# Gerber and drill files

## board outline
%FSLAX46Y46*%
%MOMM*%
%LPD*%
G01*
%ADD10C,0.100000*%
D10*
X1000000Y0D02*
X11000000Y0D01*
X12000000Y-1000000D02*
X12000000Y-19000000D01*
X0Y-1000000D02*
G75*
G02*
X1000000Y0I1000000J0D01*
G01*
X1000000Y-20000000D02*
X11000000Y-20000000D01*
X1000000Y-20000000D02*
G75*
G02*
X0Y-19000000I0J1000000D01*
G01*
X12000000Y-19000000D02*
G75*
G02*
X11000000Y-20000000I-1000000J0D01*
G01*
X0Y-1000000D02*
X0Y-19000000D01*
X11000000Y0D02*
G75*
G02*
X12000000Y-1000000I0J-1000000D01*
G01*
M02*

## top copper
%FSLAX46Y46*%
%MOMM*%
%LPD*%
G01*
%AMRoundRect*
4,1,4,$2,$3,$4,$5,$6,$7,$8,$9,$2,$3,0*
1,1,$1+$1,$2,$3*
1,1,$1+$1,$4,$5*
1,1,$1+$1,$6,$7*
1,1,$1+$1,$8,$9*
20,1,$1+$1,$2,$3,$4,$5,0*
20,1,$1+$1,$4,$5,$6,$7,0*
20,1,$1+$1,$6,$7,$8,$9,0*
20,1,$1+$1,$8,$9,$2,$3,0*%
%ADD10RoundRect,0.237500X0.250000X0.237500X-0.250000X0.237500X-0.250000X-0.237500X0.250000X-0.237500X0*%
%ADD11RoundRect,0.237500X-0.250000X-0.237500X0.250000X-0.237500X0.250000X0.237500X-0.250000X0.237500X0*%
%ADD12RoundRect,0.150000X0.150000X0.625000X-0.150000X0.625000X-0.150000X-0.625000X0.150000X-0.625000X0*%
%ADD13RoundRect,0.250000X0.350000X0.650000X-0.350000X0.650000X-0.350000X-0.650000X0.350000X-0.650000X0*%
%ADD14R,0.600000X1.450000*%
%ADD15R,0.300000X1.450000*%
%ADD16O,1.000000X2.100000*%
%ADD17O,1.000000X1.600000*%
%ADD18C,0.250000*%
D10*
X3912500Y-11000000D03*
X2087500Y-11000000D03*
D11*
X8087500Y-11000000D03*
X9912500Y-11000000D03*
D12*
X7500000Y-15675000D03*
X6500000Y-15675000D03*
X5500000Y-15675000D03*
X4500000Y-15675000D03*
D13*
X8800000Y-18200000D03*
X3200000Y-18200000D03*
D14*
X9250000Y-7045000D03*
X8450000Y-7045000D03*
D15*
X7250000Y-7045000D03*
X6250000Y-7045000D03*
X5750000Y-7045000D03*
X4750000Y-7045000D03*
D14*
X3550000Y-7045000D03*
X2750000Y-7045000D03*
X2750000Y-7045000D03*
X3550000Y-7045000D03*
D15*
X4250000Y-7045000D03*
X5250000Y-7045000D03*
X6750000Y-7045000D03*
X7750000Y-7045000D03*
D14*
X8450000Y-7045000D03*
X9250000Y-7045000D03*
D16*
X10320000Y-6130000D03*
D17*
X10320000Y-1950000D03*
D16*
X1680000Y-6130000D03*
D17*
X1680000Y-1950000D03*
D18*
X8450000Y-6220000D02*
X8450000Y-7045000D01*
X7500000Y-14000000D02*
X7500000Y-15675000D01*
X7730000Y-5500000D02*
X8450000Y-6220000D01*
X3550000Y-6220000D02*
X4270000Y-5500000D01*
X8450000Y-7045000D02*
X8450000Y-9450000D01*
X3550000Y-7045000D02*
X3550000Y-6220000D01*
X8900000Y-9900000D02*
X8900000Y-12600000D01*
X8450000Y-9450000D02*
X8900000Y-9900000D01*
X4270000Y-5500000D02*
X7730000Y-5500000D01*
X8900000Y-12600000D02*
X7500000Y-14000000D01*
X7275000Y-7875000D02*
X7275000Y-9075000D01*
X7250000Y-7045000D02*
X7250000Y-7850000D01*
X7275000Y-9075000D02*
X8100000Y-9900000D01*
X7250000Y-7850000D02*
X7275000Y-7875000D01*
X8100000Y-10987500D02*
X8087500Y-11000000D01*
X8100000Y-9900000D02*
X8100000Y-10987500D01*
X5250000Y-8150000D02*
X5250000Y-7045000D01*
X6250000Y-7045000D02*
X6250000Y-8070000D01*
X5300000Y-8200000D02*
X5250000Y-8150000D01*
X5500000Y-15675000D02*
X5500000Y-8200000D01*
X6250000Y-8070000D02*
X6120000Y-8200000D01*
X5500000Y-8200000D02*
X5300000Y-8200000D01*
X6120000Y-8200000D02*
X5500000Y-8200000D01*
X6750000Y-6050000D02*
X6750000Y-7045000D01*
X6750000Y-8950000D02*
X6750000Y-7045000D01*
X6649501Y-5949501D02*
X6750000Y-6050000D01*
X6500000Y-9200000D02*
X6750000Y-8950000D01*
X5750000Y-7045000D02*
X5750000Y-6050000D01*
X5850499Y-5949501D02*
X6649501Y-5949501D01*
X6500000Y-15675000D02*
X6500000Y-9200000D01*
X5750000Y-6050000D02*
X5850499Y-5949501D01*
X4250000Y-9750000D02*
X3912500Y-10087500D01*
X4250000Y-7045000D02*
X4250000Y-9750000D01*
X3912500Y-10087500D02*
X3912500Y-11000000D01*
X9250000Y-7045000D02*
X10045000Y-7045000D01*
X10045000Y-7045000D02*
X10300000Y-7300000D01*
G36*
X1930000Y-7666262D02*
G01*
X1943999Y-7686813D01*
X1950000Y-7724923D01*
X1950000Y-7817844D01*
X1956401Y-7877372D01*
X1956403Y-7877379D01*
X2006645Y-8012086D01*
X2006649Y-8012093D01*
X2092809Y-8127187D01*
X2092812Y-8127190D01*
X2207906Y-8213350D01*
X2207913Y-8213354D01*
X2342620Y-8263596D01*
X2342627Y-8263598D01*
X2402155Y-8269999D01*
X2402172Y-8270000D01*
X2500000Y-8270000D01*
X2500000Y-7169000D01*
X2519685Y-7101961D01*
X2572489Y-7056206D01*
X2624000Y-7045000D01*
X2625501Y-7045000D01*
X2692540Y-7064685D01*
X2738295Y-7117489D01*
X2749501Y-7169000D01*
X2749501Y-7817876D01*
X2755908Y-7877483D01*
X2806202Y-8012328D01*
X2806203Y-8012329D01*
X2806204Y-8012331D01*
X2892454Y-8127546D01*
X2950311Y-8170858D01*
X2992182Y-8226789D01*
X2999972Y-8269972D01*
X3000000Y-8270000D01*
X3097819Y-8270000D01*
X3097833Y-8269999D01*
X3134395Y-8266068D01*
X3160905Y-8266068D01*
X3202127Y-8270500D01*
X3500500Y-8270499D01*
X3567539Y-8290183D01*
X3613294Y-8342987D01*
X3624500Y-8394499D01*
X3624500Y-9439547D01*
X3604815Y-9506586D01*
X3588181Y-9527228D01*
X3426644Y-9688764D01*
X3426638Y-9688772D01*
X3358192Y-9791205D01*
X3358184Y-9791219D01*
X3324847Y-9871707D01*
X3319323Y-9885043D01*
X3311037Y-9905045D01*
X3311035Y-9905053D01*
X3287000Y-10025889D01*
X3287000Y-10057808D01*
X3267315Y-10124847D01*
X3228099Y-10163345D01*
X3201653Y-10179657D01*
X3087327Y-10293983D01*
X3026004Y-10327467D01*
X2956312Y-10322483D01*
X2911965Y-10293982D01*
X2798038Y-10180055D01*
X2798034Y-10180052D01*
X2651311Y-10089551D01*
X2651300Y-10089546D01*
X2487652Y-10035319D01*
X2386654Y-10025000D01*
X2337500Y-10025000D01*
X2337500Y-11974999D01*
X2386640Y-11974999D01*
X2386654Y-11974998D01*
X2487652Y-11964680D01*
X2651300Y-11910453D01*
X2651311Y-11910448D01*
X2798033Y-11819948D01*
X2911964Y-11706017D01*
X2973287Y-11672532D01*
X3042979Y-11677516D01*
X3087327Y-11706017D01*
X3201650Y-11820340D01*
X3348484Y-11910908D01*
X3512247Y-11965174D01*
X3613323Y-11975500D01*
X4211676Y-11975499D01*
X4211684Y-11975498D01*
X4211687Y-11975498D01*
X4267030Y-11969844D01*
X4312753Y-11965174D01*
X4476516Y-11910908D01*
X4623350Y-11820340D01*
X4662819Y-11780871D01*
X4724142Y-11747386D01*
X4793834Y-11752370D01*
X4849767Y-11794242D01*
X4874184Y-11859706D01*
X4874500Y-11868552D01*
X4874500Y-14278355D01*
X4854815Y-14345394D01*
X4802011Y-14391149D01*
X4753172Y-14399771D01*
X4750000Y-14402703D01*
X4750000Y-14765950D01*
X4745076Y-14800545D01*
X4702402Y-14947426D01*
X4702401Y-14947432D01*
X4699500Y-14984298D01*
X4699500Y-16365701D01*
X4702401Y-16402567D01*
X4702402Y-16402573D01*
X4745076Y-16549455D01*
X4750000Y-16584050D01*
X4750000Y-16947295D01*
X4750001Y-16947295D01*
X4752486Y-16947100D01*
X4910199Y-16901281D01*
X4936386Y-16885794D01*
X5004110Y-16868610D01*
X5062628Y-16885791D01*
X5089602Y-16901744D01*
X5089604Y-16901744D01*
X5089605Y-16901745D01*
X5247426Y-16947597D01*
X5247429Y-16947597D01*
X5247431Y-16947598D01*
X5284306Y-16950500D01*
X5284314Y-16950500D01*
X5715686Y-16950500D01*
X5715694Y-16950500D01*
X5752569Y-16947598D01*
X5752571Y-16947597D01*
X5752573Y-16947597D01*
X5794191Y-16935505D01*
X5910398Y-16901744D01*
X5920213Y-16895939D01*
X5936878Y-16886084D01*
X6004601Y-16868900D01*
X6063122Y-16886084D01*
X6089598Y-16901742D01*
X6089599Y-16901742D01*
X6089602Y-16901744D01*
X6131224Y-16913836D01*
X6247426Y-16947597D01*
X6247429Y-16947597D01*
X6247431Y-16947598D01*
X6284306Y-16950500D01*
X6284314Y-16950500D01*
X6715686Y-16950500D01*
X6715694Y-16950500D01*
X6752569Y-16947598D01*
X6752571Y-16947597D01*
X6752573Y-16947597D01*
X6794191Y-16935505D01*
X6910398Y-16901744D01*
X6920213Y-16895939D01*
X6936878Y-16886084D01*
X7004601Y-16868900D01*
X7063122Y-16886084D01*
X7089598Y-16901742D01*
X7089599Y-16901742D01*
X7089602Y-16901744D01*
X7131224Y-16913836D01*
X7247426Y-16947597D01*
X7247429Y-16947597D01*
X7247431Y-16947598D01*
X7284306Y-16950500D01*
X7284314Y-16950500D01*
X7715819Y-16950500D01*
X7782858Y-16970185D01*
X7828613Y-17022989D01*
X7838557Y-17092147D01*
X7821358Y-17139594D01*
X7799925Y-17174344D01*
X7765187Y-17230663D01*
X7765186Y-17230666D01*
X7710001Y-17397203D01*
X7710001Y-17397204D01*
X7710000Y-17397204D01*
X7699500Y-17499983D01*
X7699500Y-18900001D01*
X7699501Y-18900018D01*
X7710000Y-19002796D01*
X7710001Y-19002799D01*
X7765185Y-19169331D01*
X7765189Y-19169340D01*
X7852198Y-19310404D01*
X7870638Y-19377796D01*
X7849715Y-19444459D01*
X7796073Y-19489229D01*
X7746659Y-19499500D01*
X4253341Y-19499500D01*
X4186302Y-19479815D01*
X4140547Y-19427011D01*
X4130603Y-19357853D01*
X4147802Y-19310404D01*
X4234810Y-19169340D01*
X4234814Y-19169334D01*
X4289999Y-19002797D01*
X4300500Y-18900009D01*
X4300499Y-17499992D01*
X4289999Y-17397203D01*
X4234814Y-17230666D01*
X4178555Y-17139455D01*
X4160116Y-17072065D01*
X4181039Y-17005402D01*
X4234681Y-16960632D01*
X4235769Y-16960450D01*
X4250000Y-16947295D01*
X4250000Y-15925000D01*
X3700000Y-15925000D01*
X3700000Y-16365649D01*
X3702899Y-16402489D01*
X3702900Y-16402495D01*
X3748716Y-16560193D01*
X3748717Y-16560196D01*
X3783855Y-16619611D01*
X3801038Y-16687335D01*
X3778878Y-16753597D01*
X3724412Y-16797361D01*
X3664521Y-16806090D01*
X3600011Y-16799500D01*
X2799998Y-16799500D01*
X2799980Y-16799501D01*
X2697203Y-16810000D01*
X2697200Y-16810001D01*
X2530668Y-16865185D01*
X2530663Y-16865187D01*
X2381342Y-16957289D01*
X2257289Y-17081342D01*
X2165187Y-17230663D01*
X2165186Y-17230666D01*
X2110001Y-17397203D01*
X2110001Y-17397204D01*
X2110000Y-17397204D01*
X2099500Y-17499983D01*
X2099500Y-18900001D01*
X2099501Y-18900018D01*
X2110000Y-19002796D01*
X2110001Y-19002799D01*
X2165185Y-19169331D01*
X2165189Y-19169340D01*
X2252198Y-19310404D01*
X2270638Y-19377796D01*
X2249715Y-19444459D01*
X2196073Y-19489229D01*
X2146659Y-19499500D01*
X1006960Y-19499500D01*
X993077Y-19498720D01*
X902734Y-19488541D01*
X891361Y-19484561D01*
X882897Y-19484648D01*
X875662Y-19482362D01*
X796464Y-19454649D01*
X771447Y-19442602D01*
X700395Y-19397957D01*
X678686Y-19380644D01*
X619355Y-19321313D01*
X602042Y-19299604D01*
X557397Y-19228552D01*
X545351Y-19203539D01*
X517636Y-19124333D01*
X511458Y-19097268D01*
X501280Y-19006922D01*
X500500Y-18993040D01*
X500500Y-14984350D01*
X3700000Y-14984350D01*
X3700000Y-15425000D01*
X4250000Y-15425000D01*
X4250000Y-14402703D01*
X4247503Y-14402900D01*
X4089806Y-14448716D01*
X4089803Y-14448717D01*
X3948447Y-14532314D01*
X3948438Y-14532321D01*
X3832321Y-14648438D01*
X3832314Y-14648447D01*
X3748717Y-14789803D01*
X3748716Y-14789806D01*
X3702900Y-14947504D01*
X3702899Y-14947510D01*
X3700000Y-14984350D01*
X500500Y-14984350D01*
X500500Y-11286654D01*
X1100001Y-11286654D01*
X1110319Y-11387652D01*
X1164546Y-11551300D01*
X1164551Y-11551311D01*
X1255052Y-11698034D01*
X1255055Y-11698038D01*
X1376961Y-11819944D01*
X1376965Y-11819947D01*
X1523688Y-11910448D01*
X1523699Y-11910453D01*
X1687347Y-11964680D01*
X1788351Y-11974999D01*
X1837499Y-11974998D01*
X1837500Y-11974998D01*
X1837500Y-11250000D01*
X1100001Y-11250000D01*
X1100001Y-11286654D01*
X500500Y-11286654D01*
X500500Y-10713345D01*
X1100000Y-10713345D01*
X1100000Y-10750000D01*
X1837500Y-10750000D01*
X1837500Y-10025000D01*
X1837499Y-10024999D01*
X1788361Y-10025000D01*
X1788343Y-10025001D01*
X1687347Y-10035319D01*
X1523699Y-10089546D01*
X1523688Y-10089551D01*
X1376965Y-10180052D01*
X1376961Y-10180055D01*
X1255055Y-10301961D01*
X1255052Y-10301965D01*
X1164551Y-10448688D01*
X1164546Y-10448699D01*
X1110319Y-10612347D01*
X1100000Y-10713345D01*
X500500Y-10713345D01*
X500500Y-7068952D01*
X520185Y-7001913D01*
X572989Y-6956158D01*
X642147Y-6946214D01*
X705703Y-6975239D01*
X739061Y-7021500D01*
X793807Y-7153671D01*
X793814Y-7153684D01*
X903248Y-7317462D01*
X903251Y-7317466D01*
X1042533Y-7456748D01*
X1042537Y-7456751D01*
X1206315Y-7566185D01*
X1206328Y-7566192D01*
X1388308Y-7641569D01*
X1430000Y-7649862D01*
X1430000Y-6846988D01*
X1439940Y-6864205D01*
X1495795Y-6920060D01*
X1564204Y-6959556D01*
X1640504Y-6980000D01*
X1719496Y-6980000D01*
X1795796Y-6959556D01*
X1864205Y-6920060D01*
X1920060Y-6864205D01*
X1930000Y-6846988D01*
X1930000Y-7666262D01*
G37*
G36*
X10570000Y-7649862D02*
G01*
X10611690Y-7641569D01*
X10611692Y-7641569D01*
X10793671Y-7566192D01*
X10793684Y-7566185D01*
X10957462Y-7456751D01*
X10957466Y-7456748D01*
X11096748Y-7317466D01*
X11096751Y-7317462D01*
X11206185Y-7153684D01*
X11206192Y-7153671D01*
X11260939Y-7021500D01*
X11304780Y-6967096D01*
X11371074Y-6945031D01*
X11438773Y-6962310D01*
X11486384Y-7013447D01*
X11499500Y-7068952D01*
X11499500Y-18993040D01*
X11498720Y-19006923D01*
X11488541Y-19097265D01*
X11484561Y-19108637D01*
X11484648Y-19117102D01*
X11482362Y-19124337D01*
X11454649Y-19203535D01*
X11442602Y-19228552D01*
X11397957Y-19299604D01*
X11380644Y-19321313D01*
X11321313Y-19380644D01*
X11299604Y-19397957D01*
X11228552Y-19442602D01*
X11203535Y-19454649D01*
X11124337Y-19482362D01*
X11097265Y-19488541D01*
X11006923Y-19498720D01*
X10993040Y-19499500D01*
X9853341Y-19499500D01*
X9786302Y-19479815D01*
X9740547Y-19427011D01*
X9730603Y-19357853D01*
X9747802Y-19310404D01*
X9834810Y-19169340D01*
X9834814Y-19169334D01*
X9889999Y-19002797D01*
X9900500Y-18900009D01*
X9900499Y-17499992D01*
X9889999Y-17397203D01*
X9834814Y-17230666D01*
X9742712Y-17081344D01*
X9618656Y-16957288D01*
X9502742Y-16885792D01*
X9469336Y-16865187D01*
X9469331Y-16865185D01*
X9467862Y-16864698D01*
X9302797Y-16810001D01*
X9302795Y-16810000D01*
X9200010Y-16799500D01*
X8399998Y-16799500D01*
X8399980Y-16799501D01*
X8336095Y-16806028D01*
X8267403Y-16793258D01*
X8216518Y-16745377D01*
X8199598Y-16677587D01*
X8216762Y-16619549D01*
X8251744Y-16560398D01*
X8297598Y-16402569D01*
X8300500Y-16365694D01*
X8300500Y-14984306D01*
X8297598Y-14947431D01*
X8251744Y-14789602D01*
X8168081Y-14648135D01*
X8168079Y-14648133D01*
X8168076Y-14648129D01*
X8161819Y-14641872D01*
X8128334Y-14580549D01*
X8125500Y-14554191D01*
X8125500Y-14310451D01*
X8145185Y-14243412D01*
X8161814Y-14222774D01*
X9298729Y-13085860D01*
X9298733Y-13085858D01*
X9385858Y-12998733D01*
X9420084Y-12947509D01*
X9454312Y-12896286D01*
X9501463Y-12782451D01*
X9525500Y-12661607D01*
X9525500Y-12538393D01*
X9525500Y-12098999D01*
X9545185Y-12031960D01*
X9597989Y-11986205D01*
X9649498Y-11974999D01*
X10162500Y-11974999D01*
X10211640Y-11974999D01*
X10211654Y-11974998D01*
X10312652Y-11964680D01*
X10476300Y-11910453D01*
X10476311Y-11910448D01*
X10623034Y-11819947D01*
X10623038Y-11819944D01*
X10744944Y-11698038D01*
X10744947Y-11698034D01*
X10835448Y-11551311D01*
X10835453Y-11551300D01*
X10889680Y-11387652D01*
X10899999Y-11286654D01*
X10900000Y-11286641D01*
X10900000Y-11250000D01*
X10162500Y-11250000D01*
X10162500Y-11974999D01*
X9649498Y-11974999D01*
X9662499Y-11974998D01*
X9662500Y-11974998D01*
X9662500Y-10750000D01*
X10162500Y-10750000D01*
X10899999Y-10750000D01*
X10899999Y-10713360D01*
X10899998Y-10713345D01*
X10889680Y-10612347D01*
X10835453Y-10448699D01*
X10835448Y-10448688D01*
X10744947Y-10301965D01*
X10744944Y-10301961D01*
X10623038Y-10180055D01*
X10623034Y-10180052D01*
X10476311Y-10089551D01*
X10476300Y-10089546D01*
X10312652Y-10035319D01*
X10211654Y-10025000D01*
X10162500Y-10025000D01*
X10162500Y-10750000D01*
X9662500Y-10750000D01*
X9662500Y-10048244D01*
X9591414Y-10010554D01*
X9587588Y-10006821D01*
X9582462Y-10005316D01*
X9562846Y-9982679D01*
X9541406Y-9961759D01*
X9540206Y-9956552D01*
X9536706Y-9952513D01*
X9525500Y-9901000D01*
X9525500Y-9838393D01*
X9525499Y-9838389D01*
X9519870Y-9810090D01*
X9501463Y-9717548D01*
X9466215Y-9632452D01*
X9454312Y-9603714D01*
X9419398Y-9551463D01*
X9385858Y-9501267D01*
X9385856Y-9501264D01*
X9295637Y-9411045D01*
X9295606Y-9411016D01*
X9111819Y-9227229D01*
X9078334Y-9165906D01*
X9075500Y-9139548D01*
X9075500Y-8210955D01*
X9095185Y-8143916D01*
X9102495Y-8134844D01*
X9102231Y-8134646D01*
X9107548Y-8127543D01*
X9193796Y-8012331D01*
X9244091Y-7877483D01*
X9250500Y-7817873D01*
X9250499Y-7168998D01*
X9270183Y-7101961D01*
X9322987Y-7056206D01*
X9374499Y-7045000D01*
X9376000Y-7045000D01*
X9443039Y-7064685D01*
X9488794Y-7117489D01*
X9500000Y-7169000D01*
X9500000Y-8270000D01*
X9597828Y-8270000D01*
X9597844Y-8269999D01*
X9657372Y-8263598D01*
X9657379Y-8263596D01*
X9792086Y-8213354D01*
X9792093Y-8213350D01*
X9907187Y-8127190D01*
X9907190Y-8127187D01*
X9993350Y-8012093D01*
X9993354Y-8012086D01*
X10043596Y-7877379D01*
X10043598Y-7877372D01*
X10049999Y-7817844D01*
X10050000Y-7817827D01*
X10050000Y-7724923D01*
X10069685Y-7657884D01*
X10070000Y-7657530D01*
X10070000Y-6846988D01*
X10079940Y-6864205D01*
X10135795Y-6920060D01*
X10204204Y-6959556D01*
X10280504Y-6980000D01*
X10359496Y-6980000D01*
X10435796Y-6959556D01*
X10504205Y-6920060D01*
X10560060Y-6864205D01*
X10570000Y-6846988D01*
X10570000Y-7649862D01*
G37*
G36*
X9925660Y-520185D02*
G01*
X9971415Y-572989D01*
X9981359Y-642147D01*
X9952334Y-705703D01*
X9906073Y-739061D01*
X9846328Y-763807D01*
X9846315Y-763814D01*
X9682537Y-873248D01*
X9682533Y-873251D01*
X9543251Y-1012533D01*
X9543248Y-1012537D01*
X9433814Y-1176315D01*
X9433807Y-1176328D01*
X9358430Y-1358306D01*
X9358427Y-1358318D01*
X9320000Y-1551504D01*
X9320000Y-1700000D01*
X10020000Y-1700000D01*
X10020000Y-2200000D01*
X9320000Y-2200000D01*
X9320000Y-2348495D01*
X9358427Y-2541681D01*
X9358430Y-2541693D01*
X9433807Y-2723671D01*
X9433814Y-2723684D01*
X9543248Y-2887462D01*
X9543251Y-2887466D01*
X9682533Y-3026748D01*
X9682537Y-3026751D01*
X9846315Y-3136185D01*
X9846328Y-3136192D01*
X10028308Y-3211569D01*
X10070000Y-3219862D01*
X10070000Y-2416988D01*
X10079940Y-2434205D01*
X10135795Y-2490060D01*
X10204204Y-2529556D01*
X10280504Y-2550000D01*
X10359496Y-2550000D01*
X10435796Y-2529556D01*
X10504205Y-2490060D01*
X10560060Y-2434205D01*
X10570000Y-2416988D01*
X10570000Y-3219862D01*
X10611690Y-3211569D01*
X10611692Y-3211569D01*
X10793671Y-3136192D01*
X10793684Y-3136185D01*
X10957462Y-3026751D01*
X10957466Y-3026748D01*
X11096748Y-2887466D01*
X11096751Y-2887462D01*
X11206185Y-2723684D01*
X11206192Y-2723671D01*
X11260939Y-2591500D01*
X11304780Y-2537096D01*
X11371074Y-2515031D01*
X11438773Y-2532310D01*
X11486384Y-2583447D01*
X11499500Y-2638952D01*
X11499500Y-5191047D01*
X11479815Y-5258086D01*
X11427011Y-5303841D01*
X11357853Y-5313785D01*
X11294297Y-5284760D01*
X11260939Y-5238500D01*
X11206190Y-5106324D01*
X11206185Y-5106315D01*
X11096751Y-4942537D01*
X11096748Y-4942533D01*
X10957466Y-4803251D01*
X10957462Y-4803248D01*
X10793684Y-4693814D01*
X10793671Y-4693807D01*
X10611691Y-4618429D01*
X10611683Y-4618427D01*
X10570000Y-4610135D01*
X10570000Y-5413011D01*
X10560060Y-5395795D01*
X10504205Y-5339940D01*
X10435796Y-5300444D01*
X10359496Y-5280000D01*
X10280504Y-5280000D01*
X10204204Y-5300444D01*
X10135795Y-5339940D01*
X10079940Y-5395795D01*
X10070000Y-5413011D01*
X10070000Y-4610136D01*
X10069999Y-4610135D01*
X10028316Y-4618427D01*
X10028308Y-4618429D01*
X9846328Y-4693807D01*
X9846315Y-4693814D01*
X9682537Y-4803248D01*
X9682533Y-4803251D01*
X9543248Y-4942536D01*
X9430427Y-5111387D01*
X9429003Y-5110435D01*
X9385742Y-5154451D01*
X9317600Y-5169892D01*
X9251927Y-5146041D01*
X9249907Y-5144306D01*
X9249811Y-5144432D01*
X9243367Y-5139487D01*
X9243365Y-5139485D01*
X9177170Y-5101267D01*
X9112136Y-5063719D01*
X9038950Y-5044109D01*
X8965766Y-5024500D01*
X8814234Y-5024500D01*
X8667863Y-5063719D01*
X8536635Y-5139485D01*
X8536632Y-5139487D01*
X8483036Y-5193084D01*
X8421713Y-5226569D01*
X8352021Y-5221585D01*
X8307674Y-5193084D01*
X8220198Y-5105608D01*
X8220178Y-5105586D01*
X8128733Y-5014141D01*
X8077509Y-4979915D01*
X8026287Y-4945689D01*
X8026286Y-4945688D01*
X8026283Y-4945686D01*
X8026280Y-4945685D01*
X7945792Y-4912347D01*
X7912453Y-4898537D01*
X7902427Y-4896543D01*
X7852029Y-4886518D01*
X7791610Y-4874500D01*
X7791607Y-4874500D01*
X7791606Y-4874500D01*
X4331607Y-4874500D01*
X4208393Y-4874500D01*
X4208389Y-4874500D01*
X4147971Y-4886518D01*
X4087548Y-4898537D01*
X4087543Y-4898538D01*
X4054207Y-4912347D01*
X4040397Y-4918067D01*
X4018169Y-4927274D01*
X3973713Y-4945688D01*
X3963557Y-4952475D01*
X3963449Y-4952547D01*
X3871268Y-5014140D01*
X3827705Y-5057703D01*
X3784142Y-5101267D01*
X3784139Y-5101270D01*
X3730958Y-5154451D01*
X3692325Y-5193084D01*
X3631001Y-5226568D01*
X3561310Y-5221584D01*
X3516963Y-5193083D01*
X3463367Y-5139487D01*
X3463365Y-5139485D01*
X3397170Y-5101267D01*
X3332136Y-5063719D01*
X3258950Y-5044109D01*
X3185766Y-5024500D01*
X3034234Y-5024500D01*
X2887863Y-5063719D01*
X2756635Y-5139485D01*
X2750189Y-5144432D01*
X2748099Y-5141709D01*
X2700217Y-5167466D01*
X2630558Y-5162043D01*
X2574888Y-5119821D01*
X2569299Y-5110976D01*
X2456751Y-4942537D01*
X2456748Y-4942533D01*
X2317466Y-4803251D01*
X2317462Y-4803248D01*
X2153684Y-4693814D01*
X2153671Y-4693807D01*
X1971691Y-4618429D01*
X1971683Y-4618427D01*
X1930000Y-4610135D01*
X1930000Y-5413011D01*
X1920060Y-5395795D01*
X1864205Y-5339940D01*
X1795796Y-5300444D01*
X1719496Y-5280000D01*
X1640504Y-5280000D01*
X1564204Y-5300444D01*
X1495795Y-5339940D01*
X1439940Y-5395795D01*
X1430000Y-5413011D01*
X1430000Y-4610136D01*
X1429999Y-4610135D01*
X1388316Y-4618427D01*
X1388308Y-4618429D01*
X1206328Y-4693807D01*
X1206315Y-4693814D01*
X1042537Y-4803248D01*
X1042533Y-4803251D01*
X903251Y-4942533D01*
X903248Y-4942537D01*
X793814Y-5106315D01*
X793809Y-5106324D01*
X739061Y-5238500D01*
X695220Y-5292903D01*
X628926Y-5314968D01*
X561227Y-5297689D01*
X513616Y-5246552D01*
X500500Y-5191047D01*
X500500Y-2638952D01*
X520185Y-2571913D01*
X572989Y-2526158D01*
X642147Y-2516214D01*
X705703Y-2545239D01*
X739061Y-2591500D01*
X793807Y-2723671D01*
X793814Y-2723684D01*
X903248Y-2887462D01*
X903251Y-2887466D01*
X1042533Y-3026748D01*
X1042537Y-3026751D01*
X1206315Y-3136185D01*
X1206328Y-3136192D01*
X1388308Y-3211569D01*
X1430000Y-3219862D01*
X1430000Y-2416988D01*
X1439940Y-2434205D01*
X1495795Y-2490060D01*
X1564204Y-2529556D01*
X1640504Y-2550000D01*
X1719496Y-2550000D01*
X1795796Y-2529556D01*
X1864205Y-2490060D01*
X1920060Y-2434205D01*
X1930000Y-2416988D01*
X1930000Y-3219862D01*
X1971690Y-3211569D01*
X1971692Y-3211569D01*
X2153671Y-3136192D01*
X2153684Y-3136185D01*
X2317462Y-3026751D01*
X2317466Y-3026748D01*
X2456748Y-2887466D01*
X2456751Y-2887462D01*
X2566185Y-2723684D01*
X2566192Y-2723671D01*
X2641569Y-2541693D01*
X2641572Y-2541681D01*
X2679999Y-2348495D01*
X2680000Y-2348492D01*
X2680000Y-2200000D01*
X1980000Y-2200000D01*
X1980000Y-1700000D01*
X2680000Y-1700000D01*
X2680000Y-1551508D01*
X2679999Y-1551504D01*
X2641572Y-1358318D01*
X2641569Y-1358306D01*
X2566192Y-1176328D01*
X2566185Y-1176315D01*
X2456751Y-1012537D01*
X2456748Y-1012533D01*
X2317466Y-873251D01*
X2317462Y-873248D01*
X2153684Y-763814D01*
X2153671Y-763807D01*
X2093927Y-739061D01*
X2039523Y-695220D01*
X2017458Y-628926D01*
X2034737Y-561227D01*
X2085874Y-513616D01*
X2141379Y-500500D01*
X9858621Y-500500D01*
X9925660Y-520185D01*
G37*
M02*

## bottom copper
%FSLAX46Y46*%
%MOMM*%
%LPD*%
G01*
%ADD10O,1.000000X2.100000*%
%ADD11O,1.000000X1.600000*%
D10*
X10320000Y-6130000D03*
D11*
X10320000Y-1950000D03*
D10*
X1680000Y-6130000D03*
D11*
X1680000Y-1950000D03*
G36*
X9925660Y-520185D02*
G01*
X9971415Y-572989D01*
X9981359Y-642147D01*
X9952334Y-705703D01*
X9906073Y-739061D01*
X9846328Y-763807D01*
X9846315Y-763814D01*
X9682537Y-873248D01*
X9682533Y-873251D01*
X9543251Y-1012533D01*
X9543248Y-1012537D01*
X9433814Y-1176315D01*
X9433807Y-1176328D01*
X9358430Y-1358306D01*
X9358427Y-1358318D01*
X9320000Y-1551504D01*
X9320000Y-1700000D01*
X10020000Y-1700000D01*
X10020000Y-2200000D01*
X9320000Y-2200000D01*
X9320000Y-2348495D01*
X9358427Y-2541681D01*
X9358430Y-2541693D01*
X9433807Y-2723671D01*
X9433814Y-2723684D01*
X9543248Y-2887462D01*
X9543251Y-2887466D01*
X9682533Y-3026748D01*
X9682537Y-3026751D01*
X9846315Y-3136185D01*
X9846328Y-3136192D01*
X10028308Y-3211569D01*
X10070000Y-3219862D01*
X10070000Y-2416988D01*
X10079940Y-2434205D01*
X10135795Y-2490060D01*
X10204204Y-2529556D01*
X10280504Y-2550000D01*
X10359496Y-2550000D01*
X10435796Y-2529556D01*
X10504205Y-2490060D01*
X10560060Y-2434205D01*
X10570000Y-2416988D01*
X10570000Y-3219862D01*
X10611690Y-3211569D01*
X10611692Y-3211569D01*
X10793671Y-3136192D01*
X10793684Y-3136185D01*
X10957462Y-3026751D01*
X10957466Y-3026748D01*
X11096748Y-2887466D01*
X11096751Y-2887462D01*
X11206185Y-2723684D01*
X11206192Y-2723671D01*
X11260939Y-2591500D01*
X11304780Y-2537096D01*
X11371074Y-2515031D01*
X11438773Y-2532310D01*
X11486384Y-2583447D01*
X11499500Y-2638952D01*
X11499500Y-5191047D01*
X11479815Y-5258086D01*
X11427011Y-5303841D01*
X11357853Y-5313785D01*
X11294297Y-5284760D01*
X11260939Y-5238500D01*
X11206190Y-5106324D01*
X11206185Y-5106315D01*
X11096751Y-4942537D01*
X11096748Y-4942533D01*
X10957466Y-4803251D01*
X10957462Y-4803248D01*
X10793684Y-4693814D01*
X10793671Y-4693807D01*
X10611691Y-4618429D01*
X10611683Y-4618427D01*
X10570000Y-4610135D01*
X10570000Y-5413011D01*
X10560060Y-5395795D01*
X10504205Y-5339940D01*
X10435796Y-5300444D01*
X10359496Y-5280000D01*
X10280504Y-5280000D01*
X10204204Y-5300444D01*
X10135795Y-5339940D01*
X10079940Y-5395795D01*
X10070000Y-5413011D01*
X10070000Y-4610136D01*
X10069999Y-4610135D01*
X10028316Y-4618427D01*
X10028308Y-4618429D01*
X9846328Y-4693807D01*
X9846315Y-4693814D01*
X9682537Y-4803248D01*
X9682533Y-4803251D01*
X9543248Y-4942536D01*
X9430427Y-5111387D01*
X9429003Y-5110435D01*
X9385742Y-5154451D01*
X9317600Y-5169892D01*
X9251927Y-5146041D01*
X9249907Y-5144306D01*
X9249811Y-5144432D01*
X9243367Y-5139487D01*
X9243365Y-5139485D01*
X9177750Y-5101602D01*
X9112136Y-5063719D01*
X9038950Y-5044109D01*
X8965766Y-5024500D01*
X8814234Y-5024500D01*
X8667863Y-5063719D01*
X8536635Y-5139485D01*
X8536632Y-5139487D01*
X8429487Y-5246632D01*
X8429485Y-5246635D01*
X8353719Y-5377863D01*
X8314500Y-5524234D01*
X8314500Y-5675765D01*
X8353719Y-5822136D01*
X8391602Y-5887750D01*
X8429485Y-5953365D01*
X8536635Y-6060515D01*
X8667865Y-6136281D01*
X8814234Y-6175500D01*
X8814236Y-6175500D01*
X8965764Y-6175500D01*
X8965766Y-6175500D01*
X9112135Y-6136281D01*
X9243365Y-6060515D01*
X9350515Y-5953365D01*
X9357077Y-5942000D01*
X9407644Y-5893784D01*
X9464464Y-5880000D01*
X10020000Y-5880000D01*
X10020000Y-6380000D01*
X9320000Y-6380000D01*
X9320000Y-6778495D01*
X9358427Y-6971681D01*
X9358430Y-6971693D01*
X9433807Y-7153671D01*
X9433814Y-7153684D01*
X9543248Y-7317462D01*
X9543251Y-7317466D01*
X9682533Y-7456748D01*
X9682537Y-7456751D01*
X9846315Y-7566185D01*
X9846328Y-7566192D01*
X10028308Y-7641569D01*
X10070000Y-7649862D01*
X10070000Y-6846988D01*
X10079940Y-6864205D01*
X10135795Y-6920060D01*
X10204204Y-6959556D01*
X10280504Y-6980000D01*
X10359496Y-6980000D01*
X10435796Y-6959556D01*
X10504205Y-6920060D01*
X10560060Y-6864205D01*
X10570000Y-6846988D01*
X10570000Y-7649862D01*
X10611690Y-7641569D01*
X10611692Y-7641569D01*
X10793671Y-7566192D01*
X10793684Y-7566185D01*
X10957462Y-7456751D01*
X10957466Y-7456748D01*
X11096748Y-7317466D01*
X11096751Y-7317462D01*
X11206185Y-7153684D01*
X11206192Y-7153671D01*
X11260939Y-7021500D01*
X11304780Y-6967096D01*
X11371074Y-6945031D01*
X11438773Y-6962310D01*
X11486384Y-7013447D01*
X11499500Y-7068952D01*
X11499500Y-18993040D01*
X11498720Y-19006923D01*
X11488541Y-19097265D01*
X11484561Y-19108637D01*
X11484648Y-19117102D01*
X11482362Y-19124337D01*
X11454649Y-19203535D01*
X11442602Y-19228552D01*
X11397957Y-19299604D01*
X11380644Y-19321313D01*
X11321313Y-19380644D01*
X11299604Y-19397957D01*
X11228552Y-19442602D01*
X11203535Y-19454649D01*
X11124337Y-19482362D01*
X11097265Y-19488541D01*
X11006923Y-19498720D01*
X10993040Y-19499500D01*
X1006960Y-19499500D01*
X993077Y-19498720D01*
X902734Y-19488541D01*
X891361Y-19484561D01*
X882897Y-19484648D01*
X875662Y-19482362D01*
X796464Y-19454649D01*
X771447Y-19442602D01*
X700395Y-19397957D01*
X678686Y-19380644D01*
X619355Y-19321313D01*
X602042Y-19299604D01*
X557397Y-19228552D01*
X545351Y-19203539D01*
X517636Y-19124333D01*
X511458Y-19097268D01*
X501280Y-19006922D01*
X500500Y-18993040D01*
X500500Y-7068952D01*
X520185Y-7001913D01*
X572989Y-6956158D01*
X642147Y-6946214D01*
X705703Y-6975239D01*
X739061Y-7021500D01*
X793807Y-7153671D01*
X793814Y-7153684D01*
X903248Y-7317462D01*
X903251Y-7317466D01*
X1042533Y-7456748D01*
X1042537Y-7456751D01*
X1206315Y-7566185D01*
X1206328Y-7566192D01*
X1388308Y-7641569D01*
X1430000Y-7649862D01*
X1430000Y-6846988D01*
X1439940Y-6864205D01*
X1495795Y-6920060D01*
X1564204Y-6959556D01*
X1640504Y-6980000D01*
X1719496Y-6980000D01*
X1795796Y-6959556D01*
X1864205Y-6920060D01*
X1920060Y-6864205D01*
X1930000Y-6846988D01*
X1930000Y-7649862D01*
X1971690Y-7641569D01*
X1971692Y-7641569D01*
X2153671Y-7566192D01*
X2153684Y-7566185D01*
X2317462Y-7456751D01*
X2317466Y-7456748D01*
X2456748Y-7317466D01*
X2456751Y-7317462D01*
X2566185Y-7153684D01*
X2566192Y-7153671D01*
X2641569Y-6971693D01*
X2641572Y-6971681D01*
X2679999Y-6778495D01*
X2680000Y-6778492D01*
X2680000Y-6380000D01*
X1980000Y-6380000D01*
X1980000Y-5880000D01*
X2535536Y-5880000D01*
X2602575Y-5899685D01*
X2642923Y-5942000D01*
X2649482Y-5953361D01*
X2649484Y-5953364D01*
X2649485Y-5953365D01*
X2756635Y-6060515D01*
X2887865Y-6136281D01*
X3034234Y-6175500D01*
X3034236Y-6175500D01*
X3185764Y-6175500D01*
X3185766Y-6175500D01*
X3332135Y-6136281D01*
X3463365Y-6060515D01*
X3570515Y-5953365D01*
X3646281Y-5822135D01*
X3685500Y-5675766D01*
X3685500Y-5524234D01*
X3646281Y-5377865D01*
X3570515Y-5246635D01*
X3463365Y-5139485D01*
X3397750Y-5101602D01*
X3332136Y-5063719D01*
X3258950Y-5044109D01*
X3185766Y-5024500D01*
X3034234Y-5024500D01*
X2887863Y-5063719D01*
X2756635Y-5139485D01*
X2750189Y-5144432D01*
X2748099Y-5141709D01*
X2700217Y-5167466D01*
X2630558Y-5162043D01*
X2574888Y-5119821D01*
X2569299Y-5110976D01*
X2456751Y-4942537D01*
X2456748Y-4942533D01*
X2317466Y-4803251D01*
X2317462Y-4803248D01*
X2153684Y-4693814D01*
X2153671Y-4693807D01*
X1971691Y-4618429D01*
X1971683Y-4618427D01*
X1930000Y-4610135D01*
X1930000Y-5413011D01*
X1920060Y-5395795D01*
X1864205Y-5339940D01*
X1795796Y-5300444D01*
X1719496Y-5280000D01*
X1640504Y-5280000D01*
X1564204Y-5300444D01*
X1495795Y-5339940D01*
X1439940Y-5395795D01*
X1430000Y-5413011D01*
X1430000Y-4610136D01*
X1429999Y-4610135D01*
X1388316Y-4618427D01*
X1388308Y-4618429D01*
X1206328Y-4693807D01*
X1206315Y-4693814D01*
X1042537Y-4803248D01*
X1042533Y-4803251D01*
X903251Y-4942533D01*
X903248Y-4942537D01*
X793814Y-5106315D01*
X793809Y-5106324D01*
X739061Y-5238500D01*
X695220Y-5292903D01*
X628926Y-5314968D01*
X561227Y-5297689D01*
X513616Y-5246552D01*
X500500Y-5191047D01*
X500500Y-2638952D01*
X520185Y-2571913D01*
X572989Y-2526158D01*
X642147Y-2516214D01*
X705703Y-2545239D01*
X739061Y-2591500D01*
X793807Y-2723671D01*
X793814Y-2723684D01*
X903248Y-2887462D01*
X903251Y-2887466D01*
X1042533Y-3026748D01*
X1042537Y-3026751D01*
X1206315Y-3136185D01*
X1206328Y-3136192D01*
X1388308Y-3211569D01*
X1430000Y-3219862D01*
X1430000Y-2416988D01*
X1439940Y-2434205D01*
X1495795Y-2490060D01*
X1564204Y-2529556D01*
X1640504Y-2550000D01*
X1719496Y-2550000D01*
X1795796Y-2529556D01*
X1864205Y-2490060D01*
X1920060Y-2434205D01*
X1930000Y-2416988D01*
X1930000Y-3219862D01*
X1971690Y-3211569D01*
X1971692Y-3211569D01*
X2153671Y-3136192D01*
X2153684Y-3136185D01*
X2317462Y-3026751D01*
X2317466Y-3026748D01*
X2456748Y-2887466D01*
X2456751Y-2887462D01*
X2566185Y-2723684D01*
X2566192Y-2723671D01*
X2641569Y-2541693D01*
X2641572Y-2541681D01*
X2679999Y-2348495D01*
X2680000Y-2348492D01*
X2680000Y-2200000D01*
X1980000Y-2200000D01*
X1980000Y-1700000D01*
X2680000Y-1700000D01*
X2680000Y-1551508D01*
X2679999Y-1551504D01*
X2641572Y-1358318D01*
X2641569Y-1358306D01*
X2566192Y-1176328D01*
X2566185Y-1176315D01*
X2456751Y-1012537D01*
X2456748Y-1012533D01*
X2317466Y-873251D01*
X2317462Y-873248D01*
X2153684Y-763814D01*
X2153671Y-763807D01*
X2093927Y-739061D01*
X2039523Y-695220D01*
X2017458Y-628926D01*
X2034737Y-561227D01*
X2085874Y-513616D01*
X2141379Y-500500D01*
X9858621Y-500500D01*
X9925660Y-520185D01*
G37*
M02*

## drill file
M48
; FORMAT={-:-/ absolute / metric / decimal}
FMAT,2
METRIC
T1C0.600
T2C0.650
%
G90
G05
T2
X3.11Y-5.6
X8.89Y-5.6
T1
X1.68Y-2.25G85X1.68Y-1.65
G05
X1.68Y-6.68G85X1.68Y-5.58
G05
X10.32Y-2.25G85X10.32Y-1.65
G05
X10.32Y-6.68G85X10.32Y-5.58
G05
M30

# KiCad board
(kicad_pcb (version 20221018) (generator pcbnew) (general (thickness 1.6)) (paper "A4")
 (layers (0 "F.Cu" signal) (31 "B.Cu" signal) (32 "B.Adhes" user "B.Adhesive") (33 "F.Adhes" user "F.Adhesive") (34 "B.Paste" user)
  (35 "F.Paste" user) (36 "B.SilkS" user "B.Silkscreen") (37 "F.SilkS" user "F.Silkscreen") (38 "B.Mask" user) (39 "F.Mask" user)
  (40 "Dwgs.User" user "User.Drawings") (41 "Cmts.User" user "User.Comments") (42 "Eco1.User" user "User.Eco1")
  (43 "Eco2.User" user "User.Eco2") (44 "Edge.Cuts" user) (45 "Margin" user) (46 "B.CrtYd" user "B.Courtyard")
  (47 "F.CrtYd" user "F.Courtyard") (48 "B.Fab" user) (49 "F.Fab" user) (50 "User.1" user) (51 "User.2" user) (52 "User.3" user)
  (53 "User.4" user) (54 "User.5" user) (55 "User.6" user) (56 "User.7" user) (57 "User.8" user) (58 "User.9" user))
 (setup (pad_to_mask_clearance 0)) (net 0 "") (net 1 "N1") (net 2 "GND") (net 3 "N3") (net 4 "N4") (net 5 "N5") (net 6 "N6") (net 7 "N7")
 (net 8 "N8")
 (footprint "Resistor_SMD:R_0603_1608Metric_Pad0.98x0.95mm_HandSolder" (layer "F.Cu") (at 3 11 180)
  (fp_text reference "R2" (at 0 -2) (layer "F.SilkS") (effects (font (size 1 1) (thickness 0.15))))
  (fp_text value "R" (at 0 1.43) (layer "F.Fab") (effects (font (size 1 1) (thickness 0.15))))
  (pad "1" smd roundrect (at -0.9125 0 180) (size 0.975 0.95) (layers "F.Cu" "F.Paste" "F.Mask") (roundrect_rratio 0.25) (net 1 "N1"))
  (pad "2" smd roundrect (at 0.9125 0 180) (size 0.975 0.95) (layers "F.Cu" "F.Paste" "F.Mask") (roundrect_rratio 0.25) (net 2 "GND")))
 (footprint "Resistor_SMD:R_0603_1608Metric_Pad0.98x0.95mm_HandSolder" (layer "F.Cu") (at 9 11)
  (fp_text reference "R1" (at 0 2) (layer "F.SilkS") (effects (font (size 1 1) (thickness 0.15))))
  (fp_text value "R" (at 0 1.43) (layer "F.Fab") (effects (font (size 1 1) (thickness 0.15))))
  (pad "1" smd roundrect (at -0.9125 0) (size 0.975 0.95) (layers "F.Cu" "F.Paste" "F.Mask") (roundrect_rratio 0.25) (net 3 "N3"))
  (pad "2" smd roundrect (at 0.9125 0) (size 0.975 0.95) (layers "F.Cu" "F.Paste" "F.Mask") (roundrect_rratio 0.25) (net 2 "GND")))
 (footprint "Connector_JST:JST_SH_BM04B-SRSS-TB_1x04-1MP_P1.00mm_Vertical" (layer "F.Cu") (at 6 17 180)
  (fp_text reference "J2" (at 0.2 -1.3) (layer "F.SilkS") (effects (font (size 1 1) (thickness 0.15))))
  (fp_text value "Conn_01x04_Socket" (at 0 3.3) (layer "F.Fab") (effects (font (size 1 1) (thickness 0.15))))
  (pad "1" smd roundrect (at -1.5 1.325 180) (size 0.6 1.55) (layers "F.Cu" "F.Paste" "F.Mask") (roundrect_rratio 0.25) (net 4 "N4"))
  (pad "2" smd roundrect (at -0.5 1.325 180) (size 0.6 1.55) (layers "F.Cu" "F.Paste" "F.Mask") (roundrect_rratio 0.25) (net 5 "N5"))
  (pad "3" smd roundrect (at 0.5 1.325 180) (size 0.6 1.55) (layers "F.Cu" "F.Paste" "F.Mask") (roundrect_rratio 0.25) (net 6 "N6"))
  (pad "4" smd roundrect (at 1.5 1.325 180) (size 0.6 1.55) (layers "F.Cu" "F.Paste" "F.Mask") (roundrect_rratio 0.25) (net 2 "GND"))
  (pad "MP" smd roundrect (at -2.8 -1.2 180) (size 1.2 1.8) (layers "F.Cu" "F.Paste" "F.Mask") (roundrect_rratio 0.2083333333))
  (pad "MP" smd roundrect (at 2.8 -1.2 180) (size 1.2 1.8) (layers "F.Cu" "F.Paste" "F.Mask") (roundrect_rratio 0.2083333333)))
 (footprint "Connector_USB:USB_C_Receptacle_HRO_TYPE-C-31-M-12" (layer "F.Cu") (at 6 3 180)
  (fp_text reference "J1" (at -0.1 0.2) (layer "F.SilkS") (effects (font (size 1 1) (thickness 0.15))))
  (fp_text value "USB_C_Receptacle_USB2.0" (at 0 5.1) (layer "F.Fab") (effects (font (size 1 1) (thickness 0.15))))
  (pad "" np_thru_hole circle (at -2.89 -2.6 180) (size 0.65 0.65) (drill 0.65) (layers "*.Cu" "*.Mask"))
  (pad "" np_thru_hole circle (at 2.89 -2.6 180) (size 0.65 0.65) (drill 0.65) (layers "*.Cu" "*.Mask"))
  (pad "A1" smd rect (at -3.25 -4.045 180) (size 0.6 1.45) (layers "F.Cu" "F.Paste" "F.Mask") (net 2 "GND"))
  (pad "A4" smd rect (at -2.45 -4.045 180) (size 0.6 1.45) (layers "F.Cu" "F.Paste" "F.Mask") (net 4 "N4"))
  (pad "A5" smd rect (at -1.25 -4.045 180) (size 0.3 1.45) (layers "F.Cu" "F.Paste" "F.Mask") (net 3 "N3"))
  (pad "A6" smd rect (at -0.25 -4.045 180) (size 0.3 1.45) (layers "F.Cu" "F.Paste" "F.Mask") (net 6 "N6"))
  (pad "A7" smd rect (at 0.25 -4.045 180) (size 0.3 1.45) (layers "F.Cu" "F.Paste" "F.Mask") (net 5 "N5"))
  (pad "A8" smd rect (at 1.25 -4.045 180) (size 0.3 1.45) (layers "F.Cu" "F.Paste" "F.Mask") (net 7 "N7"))
  (pad "A9" smd rect (at 2.45 -4.045 180) (size 0.6 1.45) (layers "F.Cu" "F.Paste" "F.Mask") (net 4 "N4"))
  (pad "A12" smd rect (at 3.25 -4.045 180) (size 0.6 1.45) (layers "F.Cu" "F.Paste" "F.Mask") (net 2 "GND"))
  (pad "B1" smd rect (at 3.25 -4.045 180) (size 0.6 1.45) (layers "F.Cu" "F.Paste" "F.Mask") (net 2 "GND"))
  (pad "B4" smd rect (at 2.45 -4.045 180) (size 0.6 1.45) (layers "F.Cu" "F.Paste" "F.Mask") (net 4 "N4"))
  (pad "B5" smd rect (at 1.75 -4.045 180) (size 0.3 1.45) (layers "F.Cu" "F.Paste" "F.Mask") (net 1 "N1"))
  (pad "B6" smd rect (at 0.75 -4.045 180) (size 0.3 1.45) (layers "F.Cu" "F.Paste" "F.Mask") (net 6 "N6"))
  (pad "B7" smd rect (at -0.75 -4.045 180) (size 0.3 1.45) (layers "F.Cu" "F.Paste" "F.Mask") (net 5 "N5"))
  (pad "B8" smd rect (at -1.75 -4.045 180) (size 0.3 1.45) (layers "F.Cu" "F.Paste" "F.Mask") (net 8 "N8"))
  (pad "B9" smd rect (at -2.45 -4.045 180) (size 0.6 1.45) (layers "F.Cu" "F.Paste" "F.Mask") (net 4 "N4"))
  (pad "B12" smd rect (at -3.25 -4.045 180) (size 0.6 1.45) (layers "F.Cu" "F.Paste" "F.Mask") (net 2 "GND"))
  (pad "S1" thru_hole oval (at -4.32 -3.13 180) (size 1 2.1) (drill oval 0.6 1.7) (layers "*.Cu" "*.Mask") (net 2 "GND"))
  (pad "S1" thru_hole oval (at -4.32 1.05 180) (size 1 1.6) (drill oval 0.6 1.2) (layers "*.Cu" "*.Mask") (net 2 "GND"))
  (pad "S1" thru_hole oval (at 4.32 -3.13 180) (size 1 2.1) (drill oval 0.6 1.7) (layers "*.Cu" "*.Mask") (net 2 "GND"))
  (pad "S1" thru_hole oval (at 4.32 1.05 180) (size 1 1.6) (drill oval 0.6 1.2) (layers "*.Cu" "*.Mask") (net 2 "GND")))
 (gr_line (start 1 0) (end 11 0) (stroke (width 0.1) (type default)) (layer "Edge.Cuts"))
 (gr_line (start 12 1) (end 12 19) (stroke (width 0.1) (type default)) (layer "Edge.Cuts"))
 (gr_arc (start 0 1) (mid 0.292893 0.292893) (end 1 0) (stroke (width 0.1) (type default)) (layer "Edge.Cuts"))
 (gr_line (start 1 20) (end 11 20) (stroke (width 0.1) (type default)) (layer "Edge.Cuts"))
 (gr_arc (start 1 20) (mid 0.292893 19.707107) (end 0 19) (stroke (width 0.1) (type default)) (layer "Edge.Cuts"))
 (gr_arc (start 12 19) (mid 11.707107 19.707107) (end 11 20) (stroke (width 0.1) (type default)) (layer "Edge.Cuts"))
 (gr_line (start 0 1) (end 0 19) (stroke (width 0.1) (type default)) (layer "Edge.Cuts"))
 (gr_arc (start 11 0) (mid 11.707107 0.292893) (end 12 1) (stroke (width 0.1) (type default)) (layer "Edge.Cuts"))
 (segment (start 8.45 6.22) (end 8.45 7.045) (width 0.25) (layer "F.Cu") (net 4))
 (segment (start 7.5 14) (end 7.5 15.675) (width 0.25) (layer "F.Cu") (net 4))
 (segment (start 7.73 5.5) (end 8.45 6.22) (width 0.25) (layer "F.Cu") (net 4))
 (segment (start 3.55 6.22) (end 4.27 5.5) (width 0.25) (layer "F.Cu") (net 4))
 (segment (start 8.45 7.045) (end 8.45 9.45) (width 0.25) (layer "F.Cu") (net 4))
 (segment (start 3.55 7.045) (end 3.55 6.22) (width 0.25) (layer "F.Cu") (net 4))
 (segment (start 8.9 9.9) (end 8.9 12.6) (width 0.25) (layer "F.Cu") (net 4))
 (segment (start 8.45 9.45) (end 8.9 9.9) (width 0.25) (layer "F.Cu") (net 4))
 (segment (start 4.27 5.5) (end 7.73 5.5) (width 0.25) (layer "F.Cu") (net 4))
 (segment (start 8.9 12.6) (end 7.5 14) (width 0.25) (layer "F.Cu") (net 4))
 (segment (start 7.275 7.875) (end 7.275 9.075) (width 0.25) (layer "F.Cu") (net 3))
 (segment (start 7.25 7.045) (end 7.25 7.85) (width 0.25) (layer "F.Cu") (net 3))
 (segment (start 7.275 9.075) (end 8.1 9.9) (width 0.25) (layer "F.Cu") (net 3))
 (segment (start 7.25 7.85) (end 7.275 7.875) (width 0.25) (layer "F.Cu") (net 3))
 (segment (start 8.1 10.9875) (end 8.0875 11) (width 0.25) (layer "F.Cu") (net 3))
 (segment (start 8.1 9.9) (end 8.1 10.9875) (width 0.25) (layer "F.Cu") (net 3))
 (segment (start 5.25 8.15) (end 5.25 7.045) (width 0.25) (layer "F.Cu") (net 6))
 (segment (start 6.25 7.045) (end 6.25 8.07) (width 0.25) (layer "F.Cu") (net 6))
 (segment (start 5.3 8.2) (end 5.25 8.15) (width 0.25) (layer "F.Cu") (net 6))
 (segment (start 5.5 15.675) (end 5.5 8.2) (width 0.25) (layer "F.Cu") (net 6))
 (segment (start 6.25 8.07) (end 6.12 8.2) (width 0.25) (layer "F.Cu") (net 6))
 (segment (start 5.5 8.2) (end 5.3 8.2) (width 0.25) (layer "F.Cu") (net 6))
 (segment (start 6.12 8.2) (end 5.5 8.2) (width 0.25) (layer "F.Cu") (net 6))
 (segment (start 6.75 6.05) (end 6.75 7.045) (width 0.25) (layer "F.Cu") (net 5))
 (segment (start 6.75 8.95) (end 6.75 7.045) (width 0.25) (layer "F.Cu") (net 5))
 (segment (start 6.649501 5.949501) (end 6.75 6.05) (width 0.25) (layer "F.Cu") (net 5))
 (segment (start 6.5 9.2) (end 6.75 8.95) (width 0.25) (layer "F.Cu") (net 5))
 (segment (start 5.75 7.045) (end 5.75 6.05) (width 0.25) (layer "F.Cu") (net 5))
 (segment (start 5.850499 5.949501) (end 6.649501 5.949501) (width 0.25) (layer "F.Cu") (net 5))
 (segment (start 6.5 15.675) (end 6.5 9.2) (width 0.25) (layer "F.Cu") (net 5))
 (segment (start 5.75 6.05) (end 5.850499 5.949501) (width 0.25) (layer "F.Cu") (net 5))
 (segment (start 4.25 9.75) (end 3.9125 10.0875) (width 0.25) (layer "F.Cu") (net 1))
 (segment (start 4.25 7.045) (end 4.25 9.75) (width 0.25) (layer "F.Cu") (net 1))
 (segment (start 3.9125 10.0875) (end 3.9125 11) (width 0.25) (layer "F.Cu") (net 1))
 (segment (start 9.25 7.045) (end 10.045 7.045) (width 0.25) (layer "F.Cu") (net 2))
 (segment (start 10.045 7.045) (end 10.3 7.3) (width 0.25) (layer "F.Cu") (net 2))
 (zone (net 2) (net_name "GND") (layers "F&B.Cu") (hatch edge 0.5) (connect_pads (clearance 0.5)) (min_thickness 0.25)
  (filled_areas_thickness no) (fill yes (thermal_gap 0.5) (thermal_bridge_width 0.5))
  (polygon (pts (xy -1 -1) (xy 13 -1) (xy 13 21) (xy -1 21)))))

